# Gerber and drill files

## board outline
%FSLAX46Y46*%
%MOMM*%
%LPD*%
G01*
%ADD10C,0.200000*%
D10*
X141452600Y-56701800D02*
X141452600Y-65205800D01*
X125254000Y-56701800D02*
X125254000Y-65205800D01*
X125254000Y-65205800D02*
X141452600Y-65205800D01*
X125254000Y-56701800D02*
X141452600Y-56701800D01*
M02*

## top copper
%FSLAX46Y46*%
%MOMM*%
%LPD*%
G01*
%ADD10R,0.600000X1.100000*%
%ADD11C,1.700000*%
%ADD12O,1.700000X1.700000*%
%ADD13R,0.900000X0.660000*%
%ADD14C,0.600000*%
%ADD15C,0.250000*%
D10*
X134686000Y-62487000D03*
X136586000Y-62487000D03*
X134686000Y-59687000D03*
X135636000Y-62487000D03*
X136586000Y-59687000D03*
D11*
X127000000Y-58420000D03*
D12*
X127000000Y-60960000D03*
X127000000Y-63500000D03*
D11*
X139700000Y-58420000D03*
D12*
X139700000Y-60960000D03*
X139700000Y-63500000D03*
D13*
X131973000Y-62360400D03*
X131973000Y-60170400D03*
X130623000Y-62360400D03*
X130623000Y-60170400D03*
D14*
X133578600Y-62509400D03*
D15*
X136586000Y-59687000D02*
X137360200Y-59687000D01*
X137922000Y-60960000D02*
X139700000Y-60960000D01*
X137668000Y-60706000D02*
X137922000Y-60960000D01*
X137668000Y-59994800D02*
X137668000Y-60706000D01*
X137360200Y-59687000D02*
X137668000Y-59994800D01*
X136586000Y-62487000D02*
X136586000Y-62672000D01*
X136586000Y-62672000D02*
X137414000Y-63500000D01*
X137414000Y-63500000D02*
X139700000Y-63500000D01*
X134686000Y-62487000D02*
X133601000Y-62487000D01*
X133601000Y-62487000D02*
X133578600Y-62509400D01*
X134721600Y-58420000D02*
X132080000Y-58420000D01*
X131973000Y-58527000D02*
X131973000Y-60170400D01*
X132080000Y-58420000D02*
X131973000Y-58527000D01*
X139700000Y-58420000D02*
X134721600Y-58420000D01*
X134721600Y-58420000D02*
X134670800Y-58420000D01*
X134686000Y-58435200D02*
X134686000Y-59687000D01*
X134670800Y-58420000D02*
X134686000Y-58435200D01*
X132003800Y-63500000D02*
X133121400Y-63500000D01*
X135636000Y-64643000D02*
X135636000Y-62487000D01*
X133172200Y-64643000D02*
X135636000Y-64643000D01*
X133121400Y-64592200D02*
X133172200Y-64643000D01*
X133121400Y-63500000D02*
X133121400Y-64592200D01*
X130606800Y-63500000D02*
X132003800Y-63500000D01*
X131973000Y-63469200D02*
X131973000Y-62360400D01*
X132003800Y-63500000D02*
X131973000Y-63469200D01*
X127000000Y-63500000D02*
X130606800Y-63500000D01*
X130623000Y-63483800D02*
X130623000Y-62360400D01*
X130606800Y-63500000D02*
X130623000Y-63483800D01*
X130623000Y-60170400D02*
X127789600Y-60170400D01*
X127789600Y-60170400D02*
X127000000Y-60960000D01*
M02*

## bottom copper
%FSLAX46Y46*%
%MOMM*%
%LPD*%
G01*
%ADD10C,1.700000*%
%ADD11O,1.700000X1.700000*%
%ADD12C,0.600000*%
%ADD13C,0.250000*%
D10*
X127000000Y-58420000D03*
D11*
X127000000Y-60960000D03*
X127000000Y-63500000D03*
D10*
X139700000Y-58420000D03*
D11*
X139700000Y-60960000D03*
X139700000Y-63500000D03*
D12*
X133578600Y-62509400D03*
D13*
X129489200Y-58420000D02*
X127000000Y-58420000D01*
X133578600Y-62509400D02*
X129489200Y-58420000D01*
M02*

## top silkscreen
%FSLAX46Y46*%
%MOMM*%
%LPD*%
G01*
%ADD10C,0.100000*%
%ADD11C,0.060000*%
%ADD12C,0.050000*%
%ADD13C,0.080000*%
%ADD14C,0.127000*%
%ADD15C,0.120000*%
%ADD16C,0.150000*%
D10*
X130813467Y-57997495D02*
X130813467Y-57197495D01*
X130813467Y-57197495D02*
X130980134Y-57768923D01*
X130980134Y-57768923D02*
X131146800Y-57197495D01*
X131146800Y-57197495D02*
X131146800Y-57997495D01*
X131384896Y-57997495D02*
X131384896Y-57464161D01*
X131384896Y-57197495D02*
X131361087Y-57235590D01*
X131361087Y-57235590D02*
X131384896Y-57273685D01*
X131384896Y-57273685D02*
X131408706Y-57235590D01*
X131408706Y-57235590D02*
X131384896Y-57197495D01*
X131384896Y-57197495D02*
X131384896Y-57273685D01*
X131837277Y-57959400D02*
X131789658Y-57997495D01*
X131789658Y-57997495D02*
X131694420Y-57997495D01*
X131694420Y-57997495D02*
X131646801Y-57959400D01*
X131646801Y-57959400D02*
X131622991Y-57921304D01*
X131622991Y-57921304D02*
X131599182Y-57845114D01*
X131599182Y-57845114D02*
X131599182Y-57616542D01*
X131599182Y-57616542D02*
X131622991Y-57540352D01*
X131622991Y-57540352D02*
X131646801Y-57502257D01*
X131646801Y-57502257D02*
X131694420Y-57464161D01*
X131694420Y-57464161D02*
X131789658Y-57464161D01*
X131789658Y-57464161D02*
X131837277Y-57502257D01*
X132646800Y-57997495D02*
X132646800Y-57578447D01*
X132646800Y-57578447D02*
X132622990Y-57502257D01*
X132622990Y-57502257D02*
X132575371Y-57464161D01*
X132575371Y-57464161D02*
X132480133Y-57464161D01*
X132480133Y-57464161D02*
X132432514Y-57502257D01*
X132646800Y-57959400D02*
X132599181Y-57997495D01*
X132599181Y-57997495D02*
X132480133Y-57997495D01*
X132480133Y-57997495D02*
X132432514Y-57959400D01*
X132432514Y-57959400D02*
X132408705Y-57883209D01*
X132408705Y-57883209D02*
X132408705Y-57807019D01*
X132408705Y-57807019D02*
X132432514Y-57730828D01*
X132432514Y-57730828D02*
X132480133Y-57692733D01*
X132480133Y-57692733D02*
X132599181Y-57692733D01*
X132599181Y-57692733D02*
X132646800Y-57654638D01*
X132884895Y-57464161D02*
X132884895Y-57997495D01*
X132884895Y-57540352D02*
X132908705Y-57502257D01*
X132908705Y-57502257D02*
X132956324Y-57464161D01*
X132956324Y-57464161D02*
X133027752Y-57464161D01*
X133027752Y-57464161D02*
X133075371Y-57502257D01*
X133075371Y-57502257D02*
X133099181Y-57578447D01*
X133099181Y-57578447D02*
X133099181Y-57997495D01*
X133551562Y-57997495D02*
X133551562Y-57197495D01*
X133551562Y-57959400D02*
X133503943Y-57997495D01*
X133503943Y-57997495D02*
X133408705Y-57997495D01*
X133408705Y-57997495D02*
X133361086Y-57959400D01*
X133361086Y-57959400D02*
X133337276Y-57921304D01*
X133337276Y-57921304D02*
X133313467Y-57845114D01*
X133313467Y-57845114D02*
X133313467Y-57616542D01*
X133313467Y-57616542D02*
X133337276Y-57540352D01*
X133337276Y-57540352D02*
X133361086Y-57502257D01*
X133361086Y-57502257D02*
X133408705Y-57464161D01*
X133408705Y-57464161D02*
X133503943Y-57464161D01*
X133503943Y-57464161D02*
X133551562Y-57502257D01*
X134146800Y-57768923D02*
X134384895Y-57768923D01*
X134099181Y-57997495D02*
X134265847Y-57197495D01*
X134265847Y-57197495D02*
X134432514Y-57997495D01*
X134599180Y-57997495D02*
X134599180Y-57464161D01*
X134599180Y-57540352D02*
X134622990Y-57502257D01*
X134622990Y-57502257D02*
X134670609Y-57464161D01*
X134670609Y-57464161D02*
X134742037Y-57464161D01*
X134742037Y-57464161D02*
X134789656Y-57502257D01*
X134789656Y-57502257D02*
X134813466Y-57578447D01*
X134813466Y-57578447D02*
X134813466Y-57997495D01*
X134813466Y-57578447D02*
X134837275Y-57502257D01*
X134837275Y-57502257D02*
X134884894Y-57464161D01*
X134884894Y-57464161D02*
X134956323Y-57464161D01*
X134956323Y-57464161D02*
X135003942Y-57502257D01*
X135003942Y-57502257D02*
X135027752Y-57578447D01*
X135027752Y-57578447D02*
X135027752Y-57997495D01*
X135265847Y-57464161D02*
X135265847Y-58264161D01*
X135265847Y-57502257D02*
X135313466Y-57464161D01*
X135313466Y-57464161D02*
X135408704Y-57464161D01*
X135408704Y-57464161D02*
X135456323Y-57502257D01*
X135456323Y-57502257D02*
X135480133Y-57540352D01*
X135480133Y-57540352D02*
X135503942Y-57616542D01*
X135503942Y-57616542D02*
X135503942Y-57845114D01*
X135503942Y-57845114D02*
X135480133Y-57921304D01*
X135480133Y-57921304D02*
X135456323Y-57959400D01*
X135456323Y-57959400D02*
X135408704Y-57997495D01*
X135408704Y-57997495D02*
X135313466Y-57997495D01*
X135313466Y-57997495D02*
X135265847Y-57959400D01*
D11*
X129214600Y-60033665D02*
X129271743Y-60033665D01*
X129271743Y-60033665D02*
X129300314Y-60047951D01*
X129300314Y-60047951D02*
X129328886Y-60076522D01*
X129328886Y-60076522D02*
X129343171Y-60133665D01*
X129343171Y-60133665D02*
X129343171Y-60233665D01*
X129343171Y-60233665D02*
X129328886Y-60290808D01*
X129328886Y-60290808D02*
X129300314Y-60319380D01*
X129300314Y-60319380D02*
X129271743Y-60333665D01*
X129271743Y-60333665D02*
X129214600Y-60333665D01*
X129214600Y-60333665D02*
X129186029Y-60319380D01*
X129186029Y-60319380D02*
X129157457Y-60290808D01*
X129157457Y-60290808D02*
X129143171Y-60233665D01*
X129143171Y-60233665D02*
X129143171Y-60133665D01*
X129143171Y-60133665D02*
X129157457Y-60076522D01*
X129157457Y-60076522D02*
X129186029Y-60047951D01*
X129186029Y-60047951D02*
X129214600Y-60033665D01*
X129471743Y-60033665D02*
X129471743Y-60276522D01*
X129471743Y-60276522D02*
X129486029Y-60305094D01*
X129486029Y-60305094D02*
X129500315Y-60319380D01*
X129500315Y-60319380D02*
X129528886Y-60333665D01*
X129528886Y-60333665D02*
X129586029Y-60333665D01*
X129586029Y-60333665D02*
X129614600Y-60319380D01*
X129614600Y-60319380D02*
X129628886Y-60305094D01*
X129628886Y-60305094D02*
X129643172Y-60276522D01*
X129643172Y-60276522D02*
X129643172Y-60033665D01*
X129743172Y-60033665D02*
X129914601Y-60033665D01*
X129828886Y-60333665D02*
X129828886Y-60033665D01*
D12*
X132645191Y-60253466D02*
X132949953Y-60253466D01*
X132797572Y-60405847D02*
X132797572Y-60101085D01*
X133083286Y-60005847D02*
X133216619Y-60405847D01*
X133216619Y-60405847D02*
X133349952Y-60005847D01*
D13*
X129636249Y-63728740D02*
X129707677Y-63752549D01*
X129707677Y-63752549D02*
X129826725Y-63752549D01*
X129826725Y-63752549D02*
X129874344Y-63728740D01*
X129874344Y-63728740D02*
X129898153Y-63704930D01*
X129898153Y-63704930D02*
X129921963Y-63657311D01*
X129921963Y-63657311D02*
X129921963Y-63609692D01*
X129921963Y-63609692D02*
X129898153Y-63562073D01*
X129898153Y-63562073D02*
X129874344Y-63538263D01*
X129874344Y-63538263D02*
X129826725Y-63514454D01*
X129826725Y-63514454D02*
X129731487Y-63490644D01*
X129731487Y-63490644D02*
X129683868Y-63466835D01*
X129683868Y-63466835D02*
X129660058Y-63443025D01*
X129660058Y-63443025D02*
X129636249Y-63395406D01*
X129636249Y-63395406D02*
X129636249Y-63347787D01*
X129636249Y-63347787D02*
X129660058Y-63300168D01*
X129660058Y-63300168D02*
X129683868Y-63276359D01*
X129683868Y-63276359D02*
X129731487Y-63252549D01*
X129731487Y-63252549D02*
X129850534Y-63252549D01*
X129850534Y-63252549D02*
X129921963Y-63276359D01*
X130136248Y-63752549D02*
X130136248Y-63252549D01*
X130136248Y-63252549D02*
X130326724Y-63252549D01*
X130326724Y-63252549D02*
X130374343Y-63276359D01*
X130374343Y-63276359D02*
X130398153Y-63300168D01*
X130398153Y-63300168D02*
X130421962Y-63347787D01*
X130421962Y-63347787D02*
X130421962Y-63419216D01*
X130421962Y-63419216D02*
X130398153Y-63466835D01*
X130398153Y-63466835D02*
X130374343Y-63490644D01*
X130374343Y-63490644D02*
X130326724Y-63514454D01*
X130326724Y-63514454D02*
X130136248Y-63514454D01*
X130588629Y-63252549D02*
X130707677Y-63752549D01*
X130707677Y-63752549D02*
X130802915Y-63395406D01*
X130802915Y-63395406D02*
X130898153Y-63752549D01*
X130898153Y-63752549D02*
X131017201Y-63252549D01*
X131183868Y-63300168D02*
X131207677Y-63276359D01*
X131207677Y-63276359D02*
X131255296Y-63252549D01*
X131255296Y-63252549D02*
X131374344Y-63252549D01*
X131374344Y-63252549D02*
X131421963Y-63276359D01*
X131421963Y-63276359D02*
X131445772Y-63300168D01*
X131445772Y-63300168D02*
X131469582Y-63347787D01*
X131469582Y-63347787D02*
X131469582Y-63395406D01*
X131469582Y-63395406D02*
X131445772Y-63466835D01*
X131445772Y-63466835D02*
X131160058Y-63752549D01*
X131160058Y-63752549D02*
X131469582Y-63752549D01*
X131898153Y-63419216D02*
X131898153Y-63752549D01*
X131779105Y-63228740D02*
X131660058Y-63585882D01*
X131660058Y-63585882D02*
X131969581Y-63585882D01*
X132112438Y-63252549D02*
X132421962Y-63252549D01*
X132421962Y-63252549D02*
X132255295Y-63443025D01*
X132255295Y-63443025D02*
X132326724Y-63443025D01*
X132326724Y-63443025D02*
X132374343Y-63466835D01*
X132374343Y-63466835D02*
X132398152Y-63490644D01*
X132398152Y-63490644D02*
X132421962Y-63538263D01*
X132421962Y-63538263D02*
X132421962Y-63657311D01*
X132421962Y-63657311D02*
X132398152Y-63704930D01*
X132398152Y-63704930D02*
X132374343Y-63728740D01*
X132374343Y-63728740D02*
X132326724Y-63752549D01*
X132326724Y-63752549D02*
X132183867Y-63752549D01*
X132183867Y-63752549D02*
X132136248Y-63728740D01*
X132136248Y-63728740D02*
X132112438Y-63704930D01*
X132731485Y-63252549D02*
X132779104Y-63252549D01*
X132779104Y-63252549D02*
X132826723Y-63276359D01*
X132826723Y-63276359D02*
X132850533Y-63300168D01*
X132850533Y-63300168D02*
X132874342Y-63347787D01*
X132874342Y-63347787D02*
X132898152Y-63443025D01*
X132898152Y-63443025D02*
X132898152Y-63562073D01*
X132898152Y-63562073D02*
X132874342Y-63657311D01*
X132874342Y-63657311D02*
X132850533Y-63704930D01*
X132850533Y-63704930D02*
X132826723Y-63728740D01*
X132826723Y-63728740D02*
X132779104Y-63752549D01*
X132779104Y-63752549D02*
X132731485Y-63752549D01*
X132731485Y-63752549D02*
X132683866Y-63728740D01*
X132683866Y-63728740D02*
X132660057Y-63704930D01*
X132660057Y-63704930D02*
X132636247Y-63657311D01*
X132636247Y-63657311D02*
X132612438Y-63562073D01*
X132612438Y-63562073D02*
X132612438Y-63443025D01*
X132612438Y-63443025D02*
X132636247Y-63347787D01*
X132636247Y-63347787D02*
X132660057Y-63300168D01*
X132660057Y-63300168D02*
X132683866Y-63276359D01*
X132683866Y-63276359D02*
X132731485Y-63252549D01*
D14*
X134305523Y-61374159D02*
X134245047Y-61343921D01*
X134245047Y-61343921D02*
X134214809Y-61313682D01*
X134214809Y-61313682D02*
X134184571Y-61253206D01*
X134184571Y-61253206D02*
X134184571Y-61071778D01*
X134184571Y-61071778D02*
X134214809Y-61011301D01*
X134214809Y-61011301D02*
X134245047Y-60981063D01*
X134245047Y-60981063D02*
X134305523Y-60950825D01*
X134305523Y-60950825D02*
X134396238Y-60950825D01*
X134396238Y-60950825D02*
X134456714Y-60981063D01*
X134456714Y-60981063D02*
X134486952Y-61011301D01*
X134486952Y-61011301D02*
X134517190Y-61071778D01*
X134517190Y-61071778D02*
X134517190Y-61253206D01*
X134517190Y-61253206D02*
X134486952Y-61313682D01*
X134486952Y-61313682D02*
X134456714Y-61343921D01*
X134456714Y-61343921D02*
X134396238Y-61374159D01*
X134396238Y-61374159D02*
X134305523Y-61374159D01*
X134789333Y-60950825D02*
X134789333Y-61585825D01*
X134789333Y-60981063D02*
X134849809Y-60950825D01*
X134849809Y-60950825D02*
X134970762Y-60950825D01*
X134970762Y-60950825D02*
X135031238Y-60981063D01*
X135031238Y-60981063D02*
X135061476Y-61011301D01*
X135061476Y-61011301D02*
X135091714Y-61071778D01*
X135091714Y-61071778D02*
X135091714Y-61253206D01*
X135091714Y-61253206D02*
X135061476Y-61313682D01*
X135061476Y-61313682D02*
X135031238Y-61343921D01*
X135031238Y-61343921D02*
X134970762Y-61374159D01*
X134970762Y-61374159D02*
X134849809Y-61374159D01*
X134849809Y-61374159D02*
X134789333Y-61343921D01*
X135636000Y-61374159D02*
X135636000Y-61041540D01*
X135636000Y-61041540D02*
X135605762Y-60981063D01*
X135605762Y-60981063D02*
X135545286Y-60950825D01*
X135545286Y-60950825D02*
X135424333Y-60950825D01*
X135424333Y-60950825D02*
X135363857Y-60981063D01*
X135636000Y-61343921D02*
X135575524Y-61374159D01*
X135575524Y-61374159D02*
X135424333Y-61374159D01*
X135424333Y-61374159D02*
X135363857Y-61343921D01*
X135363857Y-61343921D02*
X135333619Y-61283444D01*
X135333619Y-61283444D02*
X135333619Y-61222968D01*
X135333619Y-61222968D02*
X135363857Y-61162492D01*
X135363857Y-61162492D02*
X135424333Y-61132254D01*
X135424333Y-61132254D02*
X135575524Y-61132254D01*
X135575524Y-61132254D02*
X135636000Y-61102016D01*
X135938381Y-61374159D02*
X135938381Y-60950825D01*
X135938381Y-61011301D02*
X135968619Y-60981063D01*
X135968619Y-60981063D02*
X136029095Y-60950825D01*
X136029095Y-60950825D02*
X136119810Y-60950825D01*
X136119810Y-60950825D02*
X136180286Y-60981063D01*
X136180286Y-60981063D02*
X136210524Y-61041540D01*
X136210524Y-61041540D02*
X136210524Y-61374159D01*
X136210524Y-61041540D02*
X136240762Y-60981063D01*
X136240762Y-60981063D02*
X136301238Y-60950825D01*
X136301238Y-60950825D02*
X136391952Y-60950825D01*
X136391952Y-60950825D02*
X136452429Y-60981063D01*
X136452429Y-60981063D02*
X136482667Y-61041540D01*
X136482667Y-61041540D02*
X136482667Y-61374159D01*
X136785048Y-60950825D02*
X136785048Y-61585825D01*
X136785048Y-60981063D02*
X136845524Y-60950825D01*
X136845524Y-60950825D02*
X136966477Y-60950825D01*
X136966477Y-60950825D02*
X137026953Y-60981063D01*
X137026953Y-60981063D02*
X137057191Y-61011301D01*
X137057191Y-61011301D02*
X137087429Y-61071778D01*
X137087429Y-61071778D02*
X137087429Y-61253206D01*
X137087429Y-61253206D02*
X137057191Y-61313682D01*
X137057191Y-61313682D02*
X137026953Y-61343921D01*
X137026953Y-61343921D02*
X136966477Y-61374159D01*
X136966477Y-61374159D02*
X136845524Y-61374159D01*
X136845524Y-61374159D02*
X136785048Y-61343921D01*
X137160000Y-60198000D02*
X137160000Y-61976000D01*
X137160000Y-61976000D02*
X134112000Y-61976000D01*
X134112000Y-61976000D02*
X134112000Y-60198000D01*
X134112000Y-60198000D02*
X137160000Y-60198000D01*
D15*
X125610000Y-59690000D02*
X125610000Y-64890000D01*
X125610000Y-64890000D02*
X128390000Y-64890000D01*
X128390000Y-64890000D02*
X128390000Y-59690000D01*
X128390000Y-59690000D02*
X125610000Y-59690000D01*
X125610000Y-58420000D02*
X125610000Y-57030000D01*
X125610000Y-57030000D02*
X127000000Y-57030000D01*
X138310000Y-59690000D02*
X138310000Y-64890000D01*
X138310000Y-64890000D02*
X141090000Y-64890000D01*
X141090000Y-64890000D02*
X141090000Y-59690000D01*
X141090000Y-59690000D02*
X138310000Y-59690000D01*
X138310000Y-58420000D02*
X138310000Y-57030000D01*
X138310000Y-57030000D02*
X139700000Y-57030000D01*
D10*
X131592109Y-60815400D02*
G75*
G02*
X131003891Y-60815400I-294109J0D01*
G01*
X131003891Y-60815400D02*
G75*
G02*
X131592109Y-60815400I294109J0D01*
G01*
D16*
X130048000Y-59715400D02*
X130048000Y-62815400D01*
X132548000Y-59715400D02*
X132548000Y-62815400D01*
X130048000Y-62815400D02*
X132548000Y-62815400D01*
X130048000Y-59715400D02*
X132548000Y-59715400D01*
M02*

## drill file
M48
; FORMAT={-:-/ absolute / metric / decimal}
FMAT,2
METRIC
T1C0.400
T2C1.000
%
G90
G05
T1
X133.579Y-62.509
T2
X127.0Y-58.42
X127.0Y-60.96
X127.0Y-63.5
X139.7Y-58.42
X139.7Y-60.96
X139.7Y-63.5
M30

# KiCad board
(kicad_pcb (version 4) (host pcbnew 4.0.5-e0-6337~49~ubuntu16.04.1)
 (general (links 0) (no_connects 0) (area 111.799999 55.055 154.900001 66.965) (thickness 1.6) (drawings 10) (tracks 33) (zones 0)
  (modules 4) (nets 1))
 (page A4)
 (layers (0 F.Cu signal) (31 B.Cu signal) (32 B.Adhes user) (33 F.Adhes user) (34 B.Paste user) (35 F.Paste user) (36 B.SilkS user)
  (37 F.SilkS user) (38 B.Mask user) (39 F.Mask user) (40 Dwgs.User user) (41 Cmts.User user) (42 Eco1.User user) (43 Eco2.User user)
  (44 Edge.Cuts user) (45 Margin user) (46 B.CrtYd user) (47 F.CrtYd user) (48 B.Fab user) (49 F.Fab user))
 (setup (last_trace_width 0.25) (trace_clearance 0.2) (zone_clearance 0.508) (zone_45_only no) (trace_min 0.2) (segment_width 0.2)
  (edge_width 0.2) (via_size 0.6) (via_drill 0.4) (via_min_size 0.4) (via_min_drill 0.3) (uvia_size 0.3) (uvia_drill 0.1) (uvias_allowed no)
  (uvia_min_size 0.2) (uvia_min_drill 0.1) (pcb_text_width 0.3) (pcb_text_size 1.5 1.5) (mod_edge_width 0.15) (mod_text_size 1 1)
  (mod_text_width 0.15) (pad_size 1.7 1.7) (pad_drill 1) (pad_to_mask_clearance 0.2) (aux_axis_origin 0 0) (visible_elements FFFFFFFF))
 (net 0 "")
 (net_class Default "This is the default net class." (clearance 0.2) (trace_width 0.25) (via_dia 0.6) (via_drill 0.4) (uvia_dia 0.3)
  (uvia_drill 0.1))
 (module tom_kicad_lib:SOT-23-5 (layer F.Cu) (at 135.636 61.087) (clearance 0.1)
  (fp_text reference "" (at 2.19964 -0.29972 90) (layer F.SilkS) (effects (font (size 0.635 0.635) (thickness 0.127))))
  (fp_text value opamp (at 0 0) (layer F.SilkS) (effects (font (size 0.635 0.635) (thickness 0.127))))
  (fp_line (start 1.524 -0.889) (end 1.524 0.889) (layer F.SilkS) (width 0.127))
  (fp_line (start 1.524 0.889) (end -1.524 0.889) (layer F.SilkS) (width 0.127))
  (fp_line (start -1.524 0.889) (end -1.524 -0.889) (layer F.SilkS) (width 0.127))
  (fp_line (start -1.524 -0.889) (end 1.524 -0.889) (layer F.SilkS) (width 0.127))
  (pad 1 smd rect (at -0.95 1.4) (size 0.6 1.1) (layers F.Cu F.Paste F.Mask))
  (pad 3 smd rect (at 0.95 1.4) (size 0.6 1.1) (layers F.Cu F.Paste F.Mask))
  (pad 5 smd rect (at -0.95 -1.4) (size 0.6 1.1) (layers F.Cu F.Paste F.Mask))
  (pad 2 smd rect (at 0 1.4) (size 0.6 1.1) (layers F.Cu F.Paste F.Mask))
  (pad 4 smd rect (at 0.95 -1.4) (size 0.6 1.1) (layers F.Cu F.Paste F.Mask)))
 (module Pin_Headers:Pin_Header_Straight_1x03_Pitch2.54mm (layer F.Cu) (at 127 58.42)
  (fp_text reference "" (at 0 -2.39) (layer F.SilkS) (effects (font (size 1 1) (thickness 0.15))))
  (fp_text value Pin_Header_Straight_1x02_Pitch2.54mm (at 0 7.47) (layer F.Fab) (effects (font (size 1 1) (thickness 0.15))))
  (fp_line (start -1.39 1.27) (end -1.39 6.47) (layer F.SilkS) (width 0.12))
  (fp_line (start -1.39 6.47) (end 1.39 6.47) (layer F.SilkS) (width 0.12))
  (fp_line (start 1.39 6.47) (end 1.39 1.27) (layer F.SilkS) (width 0.12))
  (fp_line (start 1.39 1.27) (end -1.39 1.27) (layer F.SilkS) (width 0.12))
  (fp_line (start -1.39 0) (end -1.39 -1.39) (layer F.SilkS) (width 0.12))
  (fp_line (start -1.39 -1.39) (end 0 -1.39) (layer F.SilkS) (width 0.12))
  (pad 1 thru_hole circle (at 0 0) (size 1.7 1.7) (drill 1) (layers *.Cu *.Mask))
  (pad 2 thru_hole oval (at 0 2.54) (size 1.7 1.7) (drill 1) (layers *.Cu *.Mask))
  (pad 3 thru_hole oval (at 0 5.08) (size 1.7 1.7) (drill 1) (layers *.Cu *.Mask)))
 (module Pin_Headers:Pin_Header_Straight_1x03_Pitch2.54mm (layer F.Cu) (at 139.7 58.42)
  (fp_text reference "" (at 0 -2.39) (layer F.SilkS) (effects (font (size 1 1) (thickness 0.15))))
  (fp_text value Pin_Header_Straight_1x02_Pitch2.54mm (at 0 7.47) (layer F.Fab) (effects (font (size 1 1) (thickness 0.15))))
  (fp_line (start -1.39 1.27) (end -1.39 6.47) (layer F.SilkS) (width 0.12))
  (fp_line (start -1.39 6.47) (end 1.39 6.47) (layer F.SilkS) (width 0.12))
  (fp_line (start 1.39 6.47) (end 1.39 1.27) (layer F.SilkS) (width 0.12))
  (fp_line (start 1.39 1.27) (end -1.39 1.27) (layer F.SilkS) (width 0.12))
  (fp_line (start -1.39 0) (end -1.39 -1.39) (layer F.SilkS) (width 0.12))
  (fp_line (start -1.39 -1.39) (end 0 -1.39) (layer F.SilkS) (width 0.12))
  (pad 1 thru_hole circle (at 0 0) (size 1.7 1.7) (drill 1) (layers *.Cu *.Mask))
  (pad 2 thru_hole oval (at 0 2.54) (size 1.7 1.7) (drill 1) (layers *.Cu *.Mask))
  (pad 3 thru_hole oval (at 0 5.08) (size 1.7 1.7) (drill 1) (layers *.Cu *.Mask)))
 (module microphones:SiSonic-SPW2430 (layer F.Cu) (at 130.048 59.7154)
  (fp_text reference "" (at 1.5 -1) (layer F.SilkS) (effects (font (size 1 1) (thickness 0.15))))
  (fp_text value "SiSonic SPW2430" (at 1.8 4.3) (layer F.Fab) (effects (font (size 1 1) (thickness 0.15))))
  (fp_circle (center 1.25 1.1) (end 1.53 1.19) (layer F.SilkS) (width 0.1))
  (fp_line (start 0 0) (end 0 3.1) (layer F.SilkS) (width 0.15))
  (fp_line (start 2.5 0) (end 2.5 3.1) (layer F.SilkS) (width 0.15))
  (fp_line (start 0 3.1) (end 2.5 3.1) (layer F.SilkS) (width 0.15))
  (fp_line (start 0 0) (end 2.5 0) (layer F.SilkS) (width 0.15))
  (pad GND smd rect (at 1.925 2.645) (size 0.9 0.66) (layers F.Cu F.Paste F.Mask))
  (pad +V smd rect (at 1.925 0.455) (size 0.9 0.66) (layers F.Cu F.Paste F.Mask))
  (pad GND smd rect (at 0.575 2.645) (size 0.9 0.66) (layers F.Cu F.Paste F.Mask))
  (pad OUT smd rect (at 0.575 0.455) (size 0.9 0.66) (layers F.Cu F.Paste F.Mask)))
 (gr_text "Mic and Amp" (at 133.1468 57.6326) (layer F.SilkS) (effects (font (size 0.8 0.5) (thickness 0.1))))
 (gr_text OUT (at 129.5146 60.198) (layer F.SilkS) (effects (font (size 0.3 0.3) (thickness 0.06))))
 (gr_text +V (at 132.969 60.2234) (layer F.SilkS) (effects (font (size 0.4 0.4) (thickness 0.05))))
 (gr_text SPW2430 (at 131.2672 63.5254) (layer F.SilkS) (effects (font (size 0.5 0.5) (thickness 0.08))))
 (gr_line (start 141.4526 56.7018) (end 141.4526 65.2058) (angle 90) (layer Edge.Cuts) (width 0.2))
 (gr_line (start 125.254 56.7018) (end 125.254 65.2058) (angle 90) (layer Edge.Cuts) (width 0.2))
 (gr_line (start 125.254 65.2058) (end 141.4526 65.2058) (angle 90) (layer Edge.Cuts) (width 0.2))
 (gr_line (start 125.254 56.7018) (end 141.4526 56.7018) (angle 90) (layer Edge.Cuts) (width 0.2))
 (segment (start 136.586 59.687) (end 137.3602 59.687) (width 0.25) (layer F.Cu) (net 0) (status 400000))
 (segment (start 137.922 60.96) (end 139.7 60.96) (width 0.25) (layer F.Cu) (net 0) (status 800000))
 (segment (start 137.668 60.706) (end 137.922 60.96) (width 0.25) (layer F.Cu) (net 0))
 (segment (start 137.668 59.9948) (end 137.668 60.706) (width 0.25) (layer F.Cu) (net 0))
 (segment (start 137.3602 59.687) (end 137.668 59.9948) (width 0.25) (layer F.Cu) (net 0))
 (segment (start 136.586 62.487) (end 136.586 62.672) (width 0.25) (layer F.Cu) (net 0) (status C00000))
 (segment (start 136.586 62.672) (end 137.414 63.5) (width 0.25) (layer F.Cu) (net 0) (status 400000))
 (segment (start 137.414 63.5) (end 139.7 63.5) (width 0.25) (layer F.Cu) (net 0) (status 800000))
 (segment (start 134.686 62.487) (end 133.601 62.487) (width 0.25) (layer F.Cu) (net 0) (status 400000))
 (segment (start 129.4892 58.42) (end 127 58.42) (width 0.25) (layer B.Cu) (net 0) (status 800000))
 (segment (start 133.5786 62.5094) (end 129.4892 58.42) (width 0.25) (layer B.Cu) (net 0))
 (via (at 133.5786 62.5094) (size 0.6) (drill 0.4) (layers F.Cu B.Cu) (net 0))
 (segment (start 133.601 62.487) (end 133.5786 62.5094) (width 0.25) (layer F.Cu) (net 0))
 (segment (start 134.7216 58.42) (end 132.08 58.42) (width 0.25) (layer F.Cu) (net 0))
 (segment (start 131.973 58.527) (end 131.973 60.1704) (width 0.25) (layer F.Cu) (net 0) (status 800000))
 (segment (start 132.08 58.42) (end 131.973 58.527) (width 0.25) (layer F.Cu) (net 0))
 (segment (start 139.7 58.42) (end 134.7216 58.42) (width 0.25) (layer F.Cu) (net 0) (status 400000))
 (segment (start 134.7216 58.42) (end 134.6708 58.42) (width 0.25) (layer F.Cu) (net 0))
 (segment (start 134.686 58.4352) (end 134.686 59.687) (width 0.25) (layer F.Cu) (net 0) (status 800000))
 (segment (start 134.6708 58.42) (end 134.686 58.4352) (width 0.25) (layer F.Cu) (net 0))
 (segment (start 132.0038 63.5) (end 133.1214 63.5) (width 0.25) (layer F.Cu) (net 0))
 (segment (start 135.636 64.643) (end 135.636 62.487) (width 0.25) (layer F.Cu) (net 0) (status 800000))
 (segment (start 133.1722 64.643) (end 135.636 64.643) (width 0.25) (layer F.Cu) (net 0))
 (segment (start 133.1214 64.5922) (end 133.1722 64.643) (width 0.25) (layer F.Cu) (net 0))
 (segment (start 133.1214 63.5) (end 133.1214 64.5922) (width 0.25) (layer F.Cu) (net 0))
 (segment (start 130.6068 63.5) (end 132.0038 63.5) (width 0.25) (layer F.Cu) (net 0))
 (segment (start 131.973 63.4692) (end 131.973 62.3604) (width 0.25) (layer F.Cu) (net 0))
 (segment (start 132.0038 63.5) (end 131.973 63.4692) (width 0.25) (layer F.Cu) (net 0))
 (segment (start 127 63.5) (end 130.6068 63.5) (width 0.25) (layer F.Cu) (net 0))
 (segment (start 130.623 63.4838) (end 130.623 62.3604) (width 0.25) (layer F.Cu) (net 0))
 (segment (start 130.6068 63.5) (end 130.623 63.4838) (width 0.25) (layer F.Cu) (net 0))
 (segment (start 130.623 60.1704) (end 127.7896 60.1704) (width 0.25) (layer F.Cu) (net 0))
 (segment (start 127.7896 60.1704) (end 127 60.96) (width 0.25) (layer F.Cu) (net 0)))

